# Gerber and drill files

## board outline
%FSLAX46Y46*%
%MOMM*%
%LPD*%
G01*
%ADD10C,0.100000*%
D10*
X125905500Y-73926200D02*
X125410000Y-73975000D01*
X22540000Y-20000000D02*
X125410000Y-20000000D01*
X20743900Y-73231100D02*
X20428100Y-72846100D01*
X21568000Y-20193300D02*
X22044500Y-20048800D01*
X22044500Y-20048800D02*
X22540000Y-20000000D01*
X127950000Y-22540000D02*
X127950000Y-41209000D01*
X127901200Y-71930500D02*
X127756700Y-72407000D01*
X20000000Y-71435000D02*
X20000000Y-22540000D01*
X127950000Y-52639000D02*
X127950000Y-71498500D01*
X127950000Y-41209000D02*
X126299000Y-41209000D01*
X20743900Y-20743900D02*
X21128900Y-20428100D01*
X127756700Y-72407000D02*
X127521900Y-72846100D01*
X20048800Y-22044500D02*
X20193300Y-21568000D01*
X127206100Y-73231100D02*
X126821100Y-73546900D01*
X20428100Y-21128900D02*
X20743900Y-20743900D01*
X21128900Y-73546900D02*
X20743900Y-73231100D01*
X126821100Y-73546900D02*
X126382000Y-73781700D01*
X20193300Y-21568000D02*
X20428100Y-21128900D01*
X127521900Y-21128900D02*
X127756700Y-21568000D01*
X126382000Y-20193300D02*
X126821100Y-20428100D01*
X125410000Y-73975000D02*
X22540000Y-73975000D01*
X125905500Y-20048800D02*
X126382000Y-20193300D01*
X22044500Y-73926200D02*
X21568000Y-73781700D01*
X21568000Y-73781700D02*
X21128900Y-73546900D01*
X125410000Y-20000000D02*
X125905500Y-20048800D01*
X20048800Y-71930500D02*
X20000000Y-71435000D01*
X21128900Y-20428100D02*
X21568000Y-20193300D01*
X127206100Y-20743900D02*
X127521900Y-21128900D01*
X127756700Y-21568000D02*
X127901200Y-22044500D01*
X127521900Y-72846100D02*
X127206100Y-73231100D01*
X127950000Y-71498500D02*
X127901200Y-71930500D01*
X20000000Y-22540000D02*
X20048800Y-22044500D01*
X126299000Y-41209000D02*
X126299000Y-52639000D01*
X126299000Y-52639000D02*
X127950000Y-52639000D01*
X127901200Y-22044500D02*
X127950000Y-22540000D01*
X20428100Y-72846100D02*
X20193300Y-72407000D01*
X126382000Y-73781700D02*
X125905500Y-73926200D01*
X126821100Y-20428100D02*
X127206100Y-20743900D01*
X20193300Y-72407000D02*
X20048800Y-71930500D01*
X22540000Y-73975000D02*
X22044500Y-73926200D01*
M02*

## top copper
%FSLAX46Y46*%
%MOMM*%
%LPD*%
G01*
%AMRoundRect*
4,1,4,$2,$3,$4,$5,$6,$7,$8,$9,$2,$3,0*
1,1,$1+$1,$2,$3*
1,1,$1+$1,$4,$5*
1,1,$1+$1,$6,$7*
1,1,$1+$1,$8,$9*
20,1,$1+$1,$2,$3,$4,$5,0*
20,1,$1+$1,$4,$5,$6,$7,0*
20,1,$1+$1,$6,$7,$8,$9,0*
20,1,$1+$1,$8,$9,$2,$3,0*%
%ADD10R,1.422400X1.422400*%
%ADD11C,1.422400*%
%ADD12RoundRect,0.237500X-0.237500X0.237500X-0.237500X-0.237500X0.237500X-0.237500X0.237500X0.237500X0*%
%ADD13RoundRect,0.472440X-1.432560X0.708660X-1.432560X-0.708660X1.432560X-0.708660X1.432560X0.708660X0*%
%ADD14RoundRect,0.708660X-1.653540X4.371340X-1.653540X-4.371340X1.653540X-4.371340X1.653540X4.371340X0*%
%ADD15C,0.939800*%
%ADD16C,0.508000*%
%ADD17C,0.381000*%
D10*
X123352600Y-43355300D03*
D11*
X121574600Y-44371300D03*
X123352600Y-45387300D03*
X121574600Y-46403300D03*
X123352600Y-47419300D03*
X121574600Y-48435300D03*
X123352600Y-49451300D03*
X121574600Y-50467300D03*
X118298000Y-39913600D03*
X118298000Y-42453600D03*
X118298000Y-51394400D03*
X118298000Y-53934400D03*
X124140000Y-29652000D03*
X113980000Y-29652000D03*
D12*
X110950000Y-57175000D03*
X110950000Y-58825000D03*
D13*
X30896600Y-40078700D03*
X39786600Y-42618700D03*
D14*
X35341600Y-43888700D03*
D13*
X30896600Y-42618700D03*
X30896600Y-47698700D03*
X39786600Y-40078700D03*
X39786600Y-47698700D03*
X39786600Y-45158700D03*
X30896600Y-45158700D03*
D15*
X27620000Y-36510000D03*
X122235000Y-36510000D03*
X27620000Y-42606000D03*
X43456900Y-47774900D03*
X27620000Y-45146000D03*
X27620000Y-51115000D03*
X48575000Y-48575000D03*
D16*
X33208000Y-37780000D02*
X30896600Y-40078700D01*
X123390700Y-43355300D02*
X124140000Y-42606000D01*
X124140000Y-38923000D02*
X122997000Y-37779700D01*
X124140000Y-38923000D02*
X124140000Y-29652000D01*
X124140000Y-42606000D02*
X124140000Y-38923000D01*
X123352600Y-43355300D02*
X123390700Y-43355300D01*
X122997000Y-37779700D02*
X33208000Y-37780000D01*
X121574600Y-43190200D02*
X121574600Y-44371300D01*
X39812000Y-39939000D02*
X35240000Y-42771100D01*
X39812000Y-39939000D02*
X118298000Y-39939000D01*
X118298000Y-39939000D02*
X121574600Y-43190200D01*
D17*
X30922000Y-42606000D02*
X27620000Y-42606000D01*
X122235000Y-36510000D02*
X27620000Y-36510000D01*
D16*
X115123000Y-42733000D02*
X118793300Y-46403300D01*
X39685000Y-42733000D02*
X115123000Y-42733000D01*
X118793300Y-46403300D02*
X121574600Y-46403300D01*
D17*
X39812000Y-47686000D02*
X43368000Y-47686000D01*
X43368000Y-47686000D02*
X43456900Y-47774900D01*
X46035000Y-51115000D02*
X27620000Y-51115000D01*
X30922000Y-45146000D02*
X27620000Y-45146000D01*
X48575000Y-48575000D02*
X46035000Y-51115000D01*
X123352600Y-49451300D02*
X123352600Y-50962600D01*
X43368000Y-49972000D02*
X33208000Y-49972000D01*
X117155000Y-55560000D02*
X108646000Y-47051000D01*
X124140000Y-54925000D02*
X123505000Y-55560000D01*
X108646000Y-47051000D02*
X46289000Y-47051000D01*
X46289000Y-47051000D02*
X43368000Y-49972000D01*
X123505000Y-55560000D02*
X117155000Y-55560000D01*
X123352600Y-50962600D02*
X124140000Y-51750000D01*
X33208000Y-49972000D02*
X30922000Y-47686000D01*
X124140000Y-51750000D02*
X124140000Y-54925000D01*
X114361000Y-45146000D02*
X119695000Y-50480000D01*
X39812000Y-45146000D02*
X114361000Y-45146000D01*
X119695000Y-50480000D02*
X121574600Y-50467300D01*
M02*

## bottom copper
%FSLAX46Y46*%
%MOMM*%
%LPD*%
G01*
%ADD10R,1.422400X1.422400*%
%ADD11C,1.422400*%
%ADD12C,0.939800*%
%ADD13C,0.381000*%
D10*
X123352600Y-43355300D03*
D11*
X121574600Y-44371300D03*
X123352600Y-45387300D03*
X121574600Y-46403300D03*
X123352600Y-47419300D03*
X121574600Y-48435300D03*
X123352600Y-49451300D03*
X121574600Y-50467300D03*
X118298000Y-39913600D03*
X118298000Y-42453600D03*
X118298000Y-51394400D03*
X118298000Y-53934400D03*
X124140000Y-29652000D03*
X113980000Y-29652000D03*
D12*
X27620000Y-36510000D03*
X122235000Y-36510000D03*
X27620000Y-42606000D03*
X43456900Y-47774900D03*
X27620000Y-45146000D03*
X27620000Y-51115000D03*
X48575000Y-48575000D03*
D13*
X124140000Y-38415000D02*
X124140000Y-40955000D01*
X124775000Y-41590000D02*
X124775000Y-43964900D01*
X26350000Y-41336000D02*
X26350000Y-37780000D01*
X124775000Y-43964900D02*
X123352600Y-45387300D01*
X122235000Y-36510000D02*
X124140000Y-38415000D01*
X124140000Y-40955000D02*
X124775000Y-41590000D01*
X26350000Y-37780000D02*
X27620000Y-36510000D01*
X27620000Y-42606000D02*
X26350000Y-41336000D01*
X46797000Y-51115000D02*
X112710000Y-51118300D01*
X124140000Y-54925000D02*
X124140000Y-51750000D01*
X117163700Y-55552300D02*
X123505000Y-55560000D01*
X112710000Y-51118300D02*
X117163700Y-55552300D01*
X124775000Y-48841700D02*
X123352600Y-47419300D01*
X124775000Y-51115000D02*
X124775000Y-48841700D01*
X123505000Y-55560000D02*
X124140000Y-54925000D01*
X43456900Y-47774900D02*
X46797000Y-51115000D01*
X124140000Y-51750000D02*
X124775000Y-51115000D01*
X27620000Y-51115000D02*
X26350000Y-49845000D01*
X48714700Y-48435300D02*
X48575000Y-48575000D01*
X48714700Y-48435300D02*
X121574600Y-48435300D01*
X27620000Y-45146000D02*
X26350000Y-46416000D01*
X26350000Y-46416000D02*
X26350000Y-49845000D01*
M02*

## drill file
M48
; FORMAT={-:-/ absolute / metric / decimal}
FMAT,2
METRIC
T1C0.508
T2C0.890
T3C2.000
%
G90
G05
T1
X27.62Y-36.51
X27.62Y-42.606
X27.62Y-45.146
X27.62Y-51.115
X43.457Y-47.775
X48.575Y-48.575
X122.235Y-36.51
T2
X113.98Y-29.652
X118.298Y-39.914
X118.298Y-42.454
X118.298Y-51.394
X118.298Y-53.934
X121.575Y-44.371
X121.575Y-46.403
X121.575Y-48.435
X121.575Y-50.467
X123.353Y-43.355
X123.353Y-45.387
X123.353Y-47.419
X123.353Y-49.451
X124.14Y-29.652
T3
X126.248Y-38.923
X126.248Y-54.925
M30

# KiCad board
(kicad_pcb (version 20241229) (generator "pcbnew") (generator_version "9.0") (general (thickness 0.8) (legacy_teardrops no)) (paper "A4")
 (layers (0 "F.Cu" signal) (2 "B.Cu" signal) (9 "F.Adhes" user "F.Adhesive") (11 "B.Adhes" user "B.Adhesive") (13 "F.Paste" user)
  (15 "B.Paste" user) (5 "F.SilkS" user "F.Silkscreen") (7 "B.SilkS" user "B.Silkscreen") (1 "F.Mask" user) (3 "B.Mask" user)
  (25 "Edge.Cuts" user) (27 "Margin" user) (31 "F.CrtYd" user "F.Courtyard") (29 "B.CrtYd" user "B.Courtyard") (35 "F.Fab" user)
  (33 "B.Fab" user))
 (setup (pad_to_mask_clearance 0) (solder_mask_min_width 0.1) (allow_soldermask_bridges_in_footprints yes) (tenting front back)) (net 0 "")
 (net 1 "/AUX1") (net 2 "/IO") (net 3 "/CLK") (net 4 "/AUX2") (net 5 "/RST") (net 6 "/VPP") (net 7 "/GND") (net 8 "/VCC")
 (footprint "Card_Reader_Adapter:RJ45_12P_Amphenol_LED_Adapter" (layer "F.Cu") (at 121.44 46.92 -90)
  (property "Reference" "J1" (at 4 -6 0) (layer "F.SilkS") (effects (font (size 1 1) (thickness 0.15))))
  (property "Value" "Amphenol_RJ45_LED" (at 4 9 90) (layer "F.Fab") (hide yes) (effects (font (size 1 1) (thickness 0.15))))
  (pad "" np_thru_hole circle (at -7.997 -4.8082 270) (size 2 2) (drill 2) (layers "*.Cu" "*.Mask"))
  (pad "" np_thru_hole circle (at 8.005 -4.8082 270) (size 2 2) (drill 2) (layers "*.Cu" "*.Mask"))
  (pad "1" thru_hole rect (at -3.5647 -1.9126 270) (size 1.4224 1.4224) (drill 0.89) (layers "*.Cu" "*.Mask") (remove_unused_layers no)
   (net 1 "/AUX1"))
  (pad "2" thru_hole circle (at -2.5487 -0.1346 270) (size 1.4224 1.4224) (drill 0.89) (layers "*.Cu" "*.Mask") (remove_unused_layers no)
   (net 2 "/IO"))
  (pad "3" thru_hole circle (at -1.5327 -1.9126 270) (size 1.4224 1.4224) (drill 0.89) (layers "*.Cu" "*.Mask") (remove_unused_layers no)
   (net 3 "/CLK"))
  (pad "4" thru_hole circle (at -0.5167 -0.1346 270) (size 1.4224 1.4224) (drill 0.89) (layers "*.Cu" "*.Mask") (remove_unused_layers no)
   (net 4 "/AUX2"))
  (pad "5" thru_hole circle (at 0.4993 -1.9126 270) (size 1.4224 1.4224) (drill 0.89) (layers "*.Cu" "*.Mask") (remove_unused_layers no)
   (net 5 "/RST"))
  (pad "6" thru_hole circle (at 1.5153 -0.1346 270) (size 1.4224 1.4224) (drill 0.89) (layers "*.Cu" "*.Mask") (remove_unused_layers no)
   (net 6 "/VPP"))
  (pad "7" thru_hole circle (at 2.5313 -1.9126 270) (size 1.4224 1.4224) (drill 0.89) (layers "*.Cu" "*.Mask") (remove_unused_layers no)
   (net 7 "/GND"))
  (pad "8" thru_hole circle (at 3.5473 -0.1346 270) (size 1.4224 1.4224) (drill 0.89) (layers "*.Cu" "*.Mask") (remove_unused_layers no)
   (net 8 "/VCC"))
  (pad "9" thru_hole circle (at -7.0064 3.142 270) (size 1.4224 1.4224) (drill 0.89) (layers "*.Cu" "*.Mask") (remove_unused_layers no)
   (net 2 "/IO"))
  (pad "10" thru_hole circle (at -4.4664 3.142 270) (size 1.4224 1.4224) (drill 0.89) (layers "*.Cu" "*.Mask") (remove_unused_layers no))
  (pad "11" thru_hole circle (at 4.4744 3.142 270) (size 1.4224 1.4224) (drill 0.89) (layers "*.Cu" "*.Mask") (remove_unused_layers no))
  (pad "12" thru_hole circle (at 7.0144 3.142 270) (size 1.4224 1.4224) (drill 0.89) (layers "*.Cu" "*.Mask") (remove_unused_layers no))
  (pad "AUX1_TAP" thru_hole circle (at -17.268 -2.7 270) (size 1.4224 1.4224) (drill 0.89) (layers "*.Cu" "*.Mask")
   (remove_unused_layers no) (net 1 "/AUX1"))
  (pad "NC_TAP" thru_hole circle (at -17.268 7.46 270) (size 1.4224 1.4224) (drill 0.89) (layers "*.Cu" "*.Mask") (remove_unused_layers no)))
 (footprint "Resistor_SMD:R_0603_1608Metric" (layer "F.Cu") (at 110.95 58 -90)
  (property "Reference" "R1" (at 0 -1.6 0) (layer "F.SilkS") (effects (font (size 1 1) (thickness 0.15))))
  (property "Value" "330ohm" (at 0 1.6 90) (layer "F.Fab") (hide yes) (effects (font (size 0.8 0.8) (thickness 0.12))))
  (pad "1" smd roundrect (at -0.825 0 270) (size 0.95 0.95) (layers "F.Cu" "F.Mask" "F.Paste") (roundrect_rratio 0.25))
  (pad "2" smd roundrect (at 0.825 0 270) (size 0.95 0.95) (layers "F.Cu" "F.Mask" "F.Paste") (roundrect_rratio 0.25)))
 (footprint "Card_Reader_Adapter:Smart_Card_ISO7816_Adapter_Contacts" (layer "F.Cu") (at 35.3416 43.8887 -90)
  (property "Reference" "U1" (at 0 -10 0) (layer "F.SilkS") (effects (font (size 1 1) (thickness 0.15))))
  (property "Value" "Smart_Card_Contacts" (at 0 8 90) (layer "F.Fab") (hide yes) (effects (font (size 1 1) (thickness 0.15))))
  (pad "AUX1" smd roundrect (at -3.81 4.445 270) (size 2.3622 3.81) (layers "F.Cu" "F.Mask") (roundrect_rratio 0.2) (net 1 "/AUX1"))
  (pad "AUX2" smd roundrect (at -1.27 -4.445 270) (size 2.3622 3.81) (layers "F.Cu" "F.Mask") (roundrect_rratio 0.2) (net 4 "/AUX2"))
  (pad "CD" smd roundrect (at 0 0 270) (size 10.16 4.7244) (layers "F.Cu" "F.Mask") (roundrect_rratio 0.15) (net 2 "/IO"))
  (pad "CLK" smd roundrect (at -1.27 4.445 270) (size 2.3622 3.81) (layers "F.Cu" "F.Mask") (roundrect_rratio 0.2) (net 3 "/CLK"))
  (pad "GND" smd roundrect (at 3.81 4.445 270) (size 2.3622 3.81) (layers "F.Cu" "F.Mask") (roundrect_rratio 0.2) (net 7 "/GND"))
  (pad "IO" smd roundrect (at -3.81 -4.445 270) (size 2.3622 3.81) (layers "F.Cu" "F.Mask") (roundrect_rratio 0.2) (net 2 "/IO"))
  (pad "RST" smd roundrect (at 3.81 -4.445 270) (size 2.3622 3.81) (layers "F.Cu" "F.Mask") (roundrect_rratio 0.2) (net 5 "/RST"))
  (pad "VCC" smd roundrect (at 1.27 -4.445 270) (size 2.3622 3.81) (layers "F.Cu" "F.Mask") (roundrect_rratio 0.2) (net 8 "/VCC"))
  (pad "VPP" smd roundrect (at 1.27 4.445 270) (size 2.3622 3.81) (layers "F.Cu" "F.Mask") (roundrect_rratio 0.2) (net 6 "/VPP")))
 (gr_line (start 125.9055 73.9262) (end 125.41 73.975) (stroke (width 0.1) (type solid)) (layer "Edge.Cuts"))
 (gr_line (start 22.54 20) (end 125.41 20) (stroke (width 0.1) (type solid)) (layer "Edge.Cuts"))
 (gr_line (start 20.7439 73.2311) (end 20.4281 72.8461) (stroke (width 0.1) (type solid)) (layer "Edge.Cuts"))
 (gr_line (start 21.568 20.1933) (end 22.0445 20.0488) (stroke (width 0.1) (type solid)) (layer "Edge.Cuts"))
 (gr_line (start 22.0445 20.0488) (end 22.54 20) (stroke (width 0.1) (type solid)) (layer "Edge.Cuts"))
 (gr_line (start 127.95 22.54) (end 127.95 41.209) (stroke (width 0.1) (type solid)) (layer "Edge.Cuts"))
 (gr_line (start 127.9012 71.9305) (end 127.7567 72.407) (stroke (width 0.1) (type solid)) (layer "Edge.Cuts"))
 (gr_line (start 20 71.435) (end 20 22.54) (stroke (width 0.1) (type solid)) (layer "Edge.Cuts"))
 (gr_line (start 127.95 52.639) (end 127.95 71.4985) (stroke (width 0.1) (type solid)) (layer "Edge.Cuts"))
 (gr_line (start 127.95 41.209) (end 126.299 41.209) (stroke (width 0.1) (type solid)) (layer "Edge.Cuts"))
 (gr_line (start 20.7439 20.7439) (end 21.1289 20.4281) (stroke (width 0.1) (type solid)) (layer "Edge.Cuts"))
 (gr_line (start 127.7567 72.407) (end 127.5219 72.8461) (stroke (width 0.1) (type solid)) (layer "Edge.Cuts"))
 (gr_line (start 20.0488 22.0445) (end 20.1933 21.568) (stroke (width 0.1) (type solid)) (layer "Edge.Cuts"))
 (gr_line (start 127.2061 73.2311) (end 126.8211 73.5469) (stroke (width 0.1) (type solid)) (layer "Edge.Cuts"))
 (gr_line (start 20.4281 21.1289) (end 20.7439 20.7439) (stroke (width 0.1) (type solid)) (layer "Edge.Cuts"))
 (gr_line (start 21.1289 73.5469) (end 20.7439 73.2311) (stroke (width 0.1) (type solid)) (layer "Edge.Cuts"))
 (gr_line (start 126.8211 73.5469) (end 126.382 73.7817) (stroke (width 0.1) (type solid)) (layer "Edge.Cuts"))
 (gr_line (start 20.1933 21.568) (end 20.4281 21.1289) (stroke (width 0.1) (type solid)) (layer "Edge.Cuts"))
 (gr_line (start 127.5219 21.1289) (end 127.7567 21.568) (stroke (width 0.1) (type solid)) (layer "Edge.Cuts"))
 (gr_line (start 126.382 20.1933) (end 126.8211 20.4281) (stroke (width 0.1) (type solid)) (layer "Edge.Cuts"))
 (gr_line (start 125.41 73.975) (end 22.54 73.975) (stroke (width 0.1) (type solid)) (layer "Edge.Cuts"))
 (gr_line (start 125.9055 20.0488) (end 126.382 20.1933) (stroke (width 0.1) (type solid)) (layer "Edge.Cuts"))
 (gr_line (start 22.0445 73.9262) (end 21.568 73.7817) (stroke (width 0.1) (type solid)) (layer "Edge.Cuts"))
 (gr_line (start 21.568 73.7817) (end 21.1289 73.5469) (stroke (width 0.1) (type solid)) (layer "Edge.Cuts"))
 (gr_line (start 125.41 20) (end 125.9055 20.0488) (stroke (width 0.1) (type solid)) (layer "Edge.Cuts"))
 (gr_line (start 20.0488 71.9305) (end 20 71.435) (stroke (width 0.1) (type solid)) (layer "Edge.Cuts"))
 (gr_line (start 21.1289 20.4281) (end 21.568 20.1933) (stroke (width 0.1) (type solid)) (layer "Edge.Cuts"))
 (gr_line (start 127.2061 20.7439) (end 127.5219 21.1289) (stroke (width 0.1) (type solid)) (layer "Edge.Cuts"))
 (gr_line (start 127.7567 21.568) (end 127.9012 22.0445) (stroke (width 0.1) (type solid)) (layer "Edge.Cuts"))
 (gr_line (start 127.5219 72.8461) (end 127.2061 73.2311) (stroke (width 0.1) (type solid)) (layer "Edge.Cuts"))
 (gr_line (start 127.95 71.4985) (end 127.9012 71.9305) (stroke (width 0.1) (type solid)) (layer "Edge.Cuts"))
 (gr_line (start 20 22.54) (end 20.0488 22.0445) (stroke (width 0.1) (type solid)) (layer "Edge.Cuts"))
 (gr_line (start 126.299 41.209) (end 126.299 52.639) (stroke (width 0.1) (type solid)) (layer "Edge.Cuts"))
 (gr_line (start 126.299 52.639) (end 127.95 52.639) (stroke (width 0.1) (type solid)) (layer "Edge.Cuts"))
 (gr_line (start 127.9012 22.0445) (end 127.95 22.54) (stroke (width 0.1) (type solid)) (layer "Edge.Cuts"))
 (gr_line (start 20.4281 72.8461) (end 20.1933 72.407) (stroke (width 0.1) (type solid)) (layer "Edge.Cuts"))
 (gr_line (start 126.382 73.7817) (end 125.9055 73.9262) (stroke (width 0.1) (type solid)) (layer "Edge.Cuts"))
 (gr_line (start 126.8211 20.4281) (end 127.2061 20.7439) (stroke (width 0.1) (type solid)) (layer "Edge.Cuts"))
 (gr_line (start 20.1933 72.407) (end 20.0488 71.9305) (stroke (width 0.1) (type solid)) (layer "Edge.Cuts"))
 (gr_line (start 22.54 73.975) (end 22.0445 73.9262) (stroke (width 0.1) (type solid)) (layer "Edge.Cuts"))
 (segment (start 33.208 37.78) (end 30.8966 40.0787) (width 0.508) (layer "F.Cu") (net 1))
 (segment (start 123.3907 43.3553) (end 124.14 42.606) (width 0.508) (layer "F.Cu") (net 1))
 (segment (start 124.14 38.923) (end 122.997 37.7797) (width 0.508) (layer "F.Cu") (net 1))
 (segment (start 124.14 38.923) (end 124.14 29.652) (width 0.508) (layer "F.Cu") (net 1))
 (segment (start 124.14 42.606) (end 124.14 38.923) (width 0.508) (layer "F.Cu") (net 1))
 (segment (start 123.3526 43.3553) (end 123.3907 43.3553) (width 0.508) (layer "F.Cu") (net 1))
 (segment (start 122.997 37.7797) (end 33.208 37.78) (width 0.508) (layer "F.Cu") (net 1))
 (segment (start 121.5746 43.1902) (end 121.5746 44.3713) (width 0.508) (layer "F.Cu") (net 2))
 (segment (start 39.812 39.939) (end 35.24 42.7711) (width 0.508) (layer "F.Cu") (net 2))
 (segment (start 39.812 39.939) (end 118.298 39.939) (width 0.508) (layer "F.Cu") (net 2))
 (segment (start 118.298 39.939) (end 121.5746 43.1902) (width 0.508) (layer "F.Cu") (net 2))
 (segment (start 30.922 42.606) (end 27.62 42.606) (width 0.381) (layer "F.Cu") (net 3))
 (segment (start 122.235 36.51) (end 27.62 36.51) (width 0.381) (layer "F.Cu") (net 3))
 (via (at 27.62 36.51) (size 0.9398) (drill 0.508) (layers "F.Cu" "B.Cu") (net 3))
 (via (at 122.235 36.51) (size 0.9398) (drill 0.508) (layers "F.Cu" "B.Cu") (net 3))
 (via (at 27.62 42.606) (size 0.9398) (drill 0.508) (layers "F.Cu" "B.Cu") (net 3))
 (segment (start 124.14 38.415) (end 124.14 40.955) (width 0.381) (layer "B.Cu") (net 3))
 (segment (start 124.775 41.59) (end 124.775 43.9649) (width 0.381) (layer "B.Cu") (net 3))
 (segment (start 26.35 41.336) (end 26.35 37.78) (width 0.381) (layer "B.Cu") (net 3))
 (segment (start 124.775 43.9649) (end 123.3526 45.3873) (width 0.381) (layer "B.Cu") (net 3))
 (segment (start 122.235 36.51) (end 124.14 38.415) (width 0.381) (layer "B.Cu") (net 3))
 (segment (start 124.14 40.955) (end 124.775 41.59) (width 0.381) (layer "B.Cu") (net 3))
 (segment (start 26.35 37.78) (end 27.62 36.51) (width 0.381) (layer "B.Cu") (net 3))
 (segment (start 27.62 42.606) (end 26.35 41.336) (width 0.381) (layer "B.Cu") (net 3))
 (segment (start 115.123 42.733) (end 118.7933 46.4033) (width 0.508) (layer "F.Cu") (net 4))
 (segment (start 39.685 42.733) (end 115.123 42.733) (width 0.508) (layer "F.Cu") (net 4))
 (segment (start 118.7933 46.4033) (end 121.5746 46.4033) (width 0.508) (layer "F.Cu") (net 4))
 (segment (start 39.812 47.686) (end 43.368 47.686) (width 0.381) (layer "F.Cu") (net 5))
 (segment (start 43.368 47.686) (end 43.4569 47.7749) (width 0.381) (layer "F.Cu") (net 5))
 (via (at 43.4569 47.7749) (size 0.9398) (drill 0.508) (layers "F.Cu" "B.Cu") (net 5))
 (segment (start 46.797 51.115) (end 112.71 51.1183) (width 0.381) (layer "B.Cu") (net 5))
 (segment (start 124.14 54.925) (end 124.14 51.75) (width 0.381) (layer "B.Cu") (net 5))
 (segment (start 117.1637 55.5523) (end 123.505 55.56) (width 0.381) (layer "B.Cu") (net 5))
 (segment (start 112.71 51.1183) (end 117.1637 55.5523) (width 0.381) (layer "B.Cu") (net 5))
 (segment (start 124.775 48.8417) (end 123.3526 47.4193) (width 0.381) (layer "B.Cu") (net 5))
 (segment (start 124.775 51.115) (end 124.775 48.8417) (width 0.381) (layer "B.Cu") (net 5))
 (segment (start 123.505 55.56) (end 124.14 54.925) (width 0.381) (layer "B.Cu") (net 5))
 (segment (start 43.4569 47.7749) (end 46.797 51.115) (width 0.381) (layer "B.Cu") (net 5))
 (segment (start 124.14 51.75) (end 124.775 51.115) (width 0.381) (layer "B.Cu") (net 5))
 (segment (start 46.035 51.115) (end 27.62 51.115) (width 0.381) (layer "F.Cu") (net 6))
 (segment (start 30.922 45.146) (end 27.62 45.146) (width 0.381) (layer "F.Cu") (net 6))
 (segment (start 48.575 48.575) (end 46.035 51.115) (width 0.381) (layer "F.Cu") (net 6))
 (via (at 27.62 45.146) (size 0.9398) (drill 0.508) (layers "F.Cu" "B.Cu") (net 6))
 (via (at 27.62 51.115) (size 0.9398) (drill 0.508) (layers "F.Cu" "B.Cu") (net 6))
 (via (at 48.575 48.575) (size 0.9398) (drill 0.508) (layers "F.Cu" "B.Cu") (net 6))
 (segment (start 27.62 51.115) (end 26.35 49.845) (width 0.381) (layer "B.Cu") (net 6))
 (segment (start 48.7147 48.4353) (end 48.575 48.575) (width 0.381) (layer "B.Cu") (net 6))
 (segment (start 48.7147 48.4353) (end 121.5746 48.4353) (width 0.381) (layer "B.Cu") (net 6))
 (segment (start 27.62 45.146) (end 26.35 46.416) (width 0.381) (layer "B.Cu") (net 6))
 (segment (start 26.35 46.416) (end 26.35 49.845) (width 0.381) (layer "B.Cu") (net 6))
 (segment (start 123.3526 49.4513) (end 123.3526 50.9626) (width 0.381) (layer "F.Cu") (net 7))
 (segment (start 43.368 49.972) (end 33.208 49.972) (width 0.381) (layer "F.Cu") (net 7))
 (segment (start 117.155 55.56) (end 108.646 47.051) (width 0.381) (layer "F.Cu") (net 7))
 (segment (start 124.14 54.925) (end 123.505 55.56) (width 0.381) (layer "F.Cu") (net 7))
 (segment (start 108.646 47.051) (end 46.289 47.051) (width 0.381) (layer "F.Cu") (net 7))
 (segment (start 46.289 47.051) (end 43.368 49.972) (width 0.381) (layer "F.Cu") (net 7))
 (segment (start 123.505 55.56) (end 117.155 55.56) (width 0.381) (layer "F.Cu") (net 7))
 (segment (start 123.3526 50.9626) (end 124.14 51.75) (width 0.381) (layer "F.Cu") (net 7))
 (segment (start 33.208 49.972) (end 30.922 47.686) (width 0.381) (layer "F.Cu") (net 7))
 (segment (start 124.14 51.75) (end 124.14 54.925) (width 0.381) (layer "F.Cu") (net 7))
 (segment (start 114.361 45.146) (end 119.695 50.48) (width 0.381) (layer "F.Cu") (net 8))
 (segment (start 39.812 45.146) (end 114.361 45.146) (width 0.381) (layer "F.Cu") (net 8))
 (segment (start 119.695 50.48) (end 121.5746 50.4673) (width 0.381) (layer "F.Cu") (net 8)))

